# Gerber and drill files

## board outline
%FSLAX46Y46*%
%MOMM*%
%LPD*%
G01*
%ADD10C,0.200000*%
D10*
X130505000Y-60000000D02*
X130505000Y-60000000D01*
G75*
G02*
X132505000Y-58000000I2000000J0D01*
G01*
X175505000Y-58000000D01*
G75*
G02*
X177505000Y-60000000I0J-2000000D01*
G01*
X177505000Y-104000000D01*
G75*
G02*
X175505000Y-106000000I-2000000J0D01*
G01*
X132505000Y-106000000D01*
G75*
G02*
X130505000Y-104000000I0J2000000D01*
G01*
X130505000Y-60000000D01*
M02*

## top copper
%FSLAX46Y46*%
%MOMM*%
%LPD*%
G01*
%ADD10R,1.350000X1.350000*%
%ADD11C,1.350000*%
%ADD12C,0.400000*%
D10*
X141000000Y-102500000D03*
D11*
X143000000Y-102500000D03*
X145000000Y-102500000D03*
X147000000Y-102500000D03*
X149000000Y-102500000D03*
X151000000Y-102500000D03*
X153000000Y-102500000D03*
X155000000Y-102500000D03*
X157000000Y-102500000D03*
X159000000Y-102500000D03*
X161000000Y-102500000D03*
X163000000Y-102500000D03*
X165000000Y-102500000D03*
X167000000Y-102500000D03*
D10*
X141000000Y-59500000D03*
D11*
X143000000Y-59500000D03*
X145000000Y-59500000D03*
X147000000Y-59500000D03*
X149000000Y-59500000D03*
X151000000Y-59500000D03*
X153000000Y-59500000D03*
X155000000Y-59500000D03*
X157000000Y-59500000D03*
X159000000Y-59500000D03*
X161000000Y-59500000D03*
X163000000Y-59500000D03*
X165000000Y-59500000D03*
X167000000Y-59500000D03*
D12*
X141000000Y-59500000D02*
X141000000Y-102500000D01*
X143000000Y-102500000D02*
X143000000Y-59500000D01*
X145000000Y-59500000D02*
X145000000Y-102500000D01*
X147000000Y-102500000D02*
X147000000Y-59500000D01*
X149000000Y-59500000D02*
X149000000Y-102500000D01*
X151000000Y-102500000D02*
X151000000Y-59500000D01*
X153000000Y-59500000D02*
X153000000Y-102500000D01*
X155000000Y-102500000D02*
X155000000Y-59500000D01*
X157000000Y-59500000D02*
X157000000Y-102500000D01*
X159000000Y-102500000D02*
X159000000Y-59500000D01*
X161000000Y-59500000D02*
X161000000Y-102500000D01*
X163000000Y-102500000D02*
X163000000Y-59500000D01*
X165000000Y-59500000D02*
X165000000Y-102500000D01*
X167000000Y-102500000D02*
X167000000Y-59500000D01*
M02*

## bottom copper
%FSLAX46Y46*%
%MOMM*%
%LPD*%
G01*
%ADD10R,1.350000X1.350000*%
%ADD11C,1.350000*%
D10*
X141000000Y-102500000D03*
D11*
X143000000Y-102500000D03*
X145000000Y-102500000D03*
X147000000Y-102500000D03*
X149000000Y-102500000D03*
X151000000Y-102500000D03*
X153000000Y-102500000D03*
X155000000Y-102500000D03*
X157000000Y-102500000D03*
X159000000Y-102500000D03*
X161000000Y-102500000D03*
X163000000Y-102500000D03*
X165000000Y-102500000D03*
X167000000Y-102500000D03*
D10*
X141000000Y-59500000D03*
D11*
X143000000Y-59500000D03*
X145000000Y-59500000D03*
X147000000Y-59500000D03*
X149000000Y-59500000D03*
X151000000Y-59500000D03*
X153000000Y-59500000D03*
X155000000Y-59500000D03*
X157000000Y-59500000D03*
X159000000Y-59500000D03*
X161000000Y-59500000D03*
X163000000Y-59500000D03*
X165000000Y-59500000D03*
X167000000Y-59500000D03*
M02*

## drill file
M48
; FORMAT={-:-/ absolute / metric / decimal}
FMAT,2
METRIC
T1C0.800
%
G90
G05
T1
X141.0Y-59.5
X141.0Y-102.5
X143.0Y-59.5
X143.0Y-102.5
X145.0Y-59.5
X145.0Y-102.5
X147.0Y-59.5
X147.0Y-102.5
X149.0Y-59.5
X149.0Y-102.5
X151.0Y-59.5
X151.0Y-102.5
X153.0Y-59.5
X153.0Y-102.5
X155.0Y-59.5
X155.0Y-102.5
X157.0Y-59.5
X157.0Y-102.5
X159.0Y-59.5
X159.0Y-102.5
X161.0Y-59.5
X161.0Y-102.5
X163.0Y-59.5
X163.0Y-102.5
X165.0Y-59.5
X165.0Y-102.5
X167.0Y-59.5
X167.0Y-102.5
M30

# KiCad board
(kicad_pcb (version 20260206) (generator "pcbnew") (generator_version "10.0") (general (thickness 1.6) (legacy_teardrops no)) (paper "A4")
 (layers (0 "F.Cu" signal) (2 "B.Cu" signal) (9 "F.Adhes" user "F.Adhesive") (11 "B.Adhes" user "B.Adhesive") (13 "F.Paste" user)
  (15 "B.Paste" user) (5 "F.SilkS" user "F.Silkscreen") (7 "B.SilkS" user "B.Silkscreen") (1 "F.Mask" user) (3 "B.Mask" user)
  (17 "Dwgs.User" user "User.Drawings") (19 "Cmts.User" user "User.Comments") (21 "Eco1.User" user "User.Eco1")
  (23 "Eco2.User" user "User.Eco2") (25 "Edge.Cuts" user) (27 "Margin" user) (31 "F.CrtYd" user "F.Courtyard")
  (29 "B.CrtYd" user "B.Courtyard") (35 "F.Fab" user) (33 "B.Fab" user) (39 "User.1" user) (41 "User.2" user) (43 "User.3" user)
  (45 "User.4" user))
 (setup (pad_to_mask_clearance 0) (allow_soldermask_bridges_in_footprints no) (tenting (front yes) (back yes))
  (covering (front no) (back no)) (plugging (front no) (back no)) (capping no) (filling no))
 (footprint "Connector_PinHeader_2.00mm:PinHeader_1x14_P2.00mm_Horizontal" (layer "F.Cu") (at 167 102.5 -90)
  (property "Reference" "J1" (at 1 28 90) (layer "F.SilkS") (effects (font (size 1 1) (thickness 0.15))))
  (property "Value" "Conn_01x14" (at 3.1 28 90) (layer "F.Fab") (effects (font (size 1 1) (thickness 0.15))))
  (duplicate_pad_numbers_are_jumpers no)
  (pad "1" thru_hole rect (at 0 26 270) (size 1.35 1.35) (drill 0.8) (layers "*.Cu" "*.Mask") (remove_unused_layers no)
   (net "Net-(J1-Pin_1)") (thermal_bridge_angle 45))
  (pad "2" thru_hole circle (at 0 24 270) (size 1.35 1.35) (drill 0.8) (layers "*.Cu" "*.Mask") (remove_unused_layers no)
   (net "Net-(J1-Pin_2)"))
  (pad "3" thru_hole circle (at 0 22 270) (size 1.35 1.35) (drill 0.8) (layers "*.Cu" "*.Mask") (remove_unused_layers no)
   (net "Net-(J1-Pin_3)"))
  (pad "4" thru_hole circle (at 0 20 270) (size 1.35 1.35) (drill 0.8) (layers "*.Cu" "*.Mask") (remove_unused_layers no)
   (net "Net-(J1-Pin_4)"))
  (pad "5" thru_hole circle (at 0 18 270) (size 1.35 1.35) (drill 0.8) (layers "*.Cu" "*.Mask") (remove_unused_layers no)
   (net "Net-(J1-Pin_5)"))
  (pad "6" thru_hole circle (at 0 16 270) (size 1.35 1.35) (drill 0.8) (layers "*.Cu" "*.Mask") (remove_unused_layers no)
   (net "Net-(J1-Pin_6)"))
  (pad "7" thru_hole circle (at 0 14 270) (size 1.35 1.35) (drill 0.8) (layers "*.Cu" "*.Mask") (remove_unused_layers no)
   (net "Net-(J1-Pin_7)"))
  (pad "8" thru_hole circle (at 0 12 270) (size 1.35 1.35) (drill 0.8) (layers "*.Cu" "*.Mask") (remove_unused_layers no)
   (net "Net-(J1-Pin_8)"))
  (pad "9" thru_hole circle (at 0 10 270) (size 1.35 1.35) (drill 0.8) (layers "*.Cu" "*.Mask") (remove_unused_layers no)
   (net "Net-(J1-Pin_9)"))
  (pad "10" thru_hole circle (at 0 8 270) (size 1.35 1.35) (drill 0.8) (layers "*.Cu" "*.Mask") (remove_unused_layers no)
   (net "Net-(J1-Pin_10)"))
  (pad "11" thru_hole circle (at 0 6 270) (size 1.35 1.35) (drill 0.8) (layers "*.Cu" "*.Mask") (remove_unused_layers no)
   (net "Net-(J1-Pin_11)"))
  (pad "12" thru_hole circle (at 0 4 270) (size 1.35 1.35) (drill 0.8) (layers "*.Cu" "*.Mask") (remove_unused_layers no)
   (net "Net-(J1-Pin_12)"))
  (pad "13" thru_hole circle (at 0 2 270) (size 1.35 1.35) (drill 0.8) (layers "*.Cu" "*.Mask") (remove_unused_layers no)
   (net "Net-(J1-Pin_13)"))
  (pad "14" thru_hole circle (at 0 0 270) (size 1.35 1.35) (drill 0.8) (layers "*.Cu" "*.Mask") (remove_unused_layers no)
   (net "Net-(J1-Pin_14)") (thermal_bridge_angle 90)))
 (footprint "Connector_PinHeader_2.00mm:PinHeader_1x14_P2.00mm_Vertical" (layer "F.Cu") (at 141 59.5 90)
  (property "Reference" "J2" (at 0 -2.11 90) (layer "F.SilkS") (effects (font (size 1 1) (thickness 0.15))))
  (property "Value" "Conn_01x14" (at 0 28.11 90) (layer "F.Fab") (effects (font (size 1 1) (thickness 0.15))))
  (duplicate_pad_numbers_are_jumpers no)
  (pad "1" thru_hole rect (at 0 0 90) (size 1.35 1.35) (drill 0.8) (layers "*.Cu" "*.Mask") (remove_unused_layers no) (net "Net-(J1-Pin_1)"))
  (pad "2" thru_hole circle (at 0 2 90) (size 1.35 1.35) (drill 0.8) (layers "*.Cu" "*.Mask") (remove_unused_layers no)
   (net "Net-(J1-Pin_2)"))
  (pad "3" thru_hole circle (at 0 4 90) (size 1.35 1.35) (drill 0.8) (layers "*.Cu" "*.Mask") (remove_unused_layers no)
   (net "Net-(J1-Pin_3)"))
  (pad "4" thru_hole circle (at 0 6 90) (size 1.35 1.35) (drill 0.8) (layers "*.Cu" "*.Mask") (remove_unused_layers no)
   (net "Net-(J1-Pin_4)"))
  (pad "5" thru_hole circle (at 0 8 90) (size 1.35 1.35) (drill 0.8) (layers "*.Cu" "*.Mask") (remove_unused_layers no)
   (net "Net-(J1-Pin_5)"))
  (pad "6" thru_hole circle (at 0 10 90) (size 1.35 1.35) (drill 0.8) (layers "*.Cu" "*.Mask") (remove_unused_layers no)
   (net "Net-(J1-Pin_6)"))
  (pad "7" thru_hole circle (at 0 12 90) (size 1.35 1.35) (drill 0.8) (layers "*.Cu" "*.Mask") (remove_unused_layers no)
   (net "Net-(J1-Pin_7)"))
  (pad "8" thru_hole circle (at 0 14 90) (size 1.35 1.35) (drill 0.8) (layers "*.Cu" "*.Mask") (remove_unused_layers no)
   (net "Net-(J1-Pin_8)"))
  (pad "9" thru_hole circle (at 0 16 90) (size 1.35 1.35) (drill 0.8) (layers "*.Cu" "*.Mask") (remove_unused_layers no)
   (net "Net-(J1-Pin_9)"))
  (pad "10" thru_hole circle (at 0 18 90) (size 1.35 1.35) (drill 0.8) (layers "*.Cu" "*.Mask") (remove_unused_layers no)
   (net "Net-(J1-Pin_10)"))
  (pad "11" thru_hole circle (at 0 20 90) (size 1.35 1.35) (drill 0.8) (layers "*.Cu" "*.Mask") (remove_unused_layers no)
   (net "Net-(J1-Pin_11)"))
  (pad "12" thru_hole circle (at 0 22 90) (size 1.35 1.35) (drill 0.8) (layers "*.Cu" "*.Mask") (remove_unused_layers no)
   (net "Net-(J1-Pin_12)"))
  (pad "13" thru_hole circle (at 0 24 90) (size 1.35 1.35) (drill 0.8) (layers "*.Cu" "*.Mask") (remove_unused_layers no)
   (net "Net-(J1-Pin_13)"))
  (pad "14" thru_hole circle (at 0 26 90) (size 1.35 1.35) (drill 0.8) (layers "*.Cu" "*.Mask") (remove_unused_layers no)
   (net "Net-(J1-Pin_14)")))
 (gr_rect (start 130.505 58) (end 177.505 106) (radius 2) (stroke (width 0.2) (type solid)) (fill no) (layer "Edge.Cuts"))
 (segment (start 141 59.5) (end 141 102.5) (width 0.4) (layer "F.Cu") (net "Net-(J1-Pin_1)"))
 (segment (start 143 102.5) (end 143 59.5) (width 0.4) (layer "F.Cu") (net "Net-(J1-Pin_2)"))
 (segment (start 145 59.5) (end 145 102.5) (width 0.4) (layer "F.Cu") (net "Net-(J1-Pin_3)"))
 (segment (start 147 102.5) (end 147 59.5) (width 0.4) (layer "F.Cu") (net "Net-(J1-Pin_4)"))
 (segment (start 149 59.5) (end 149 102.5) (width 0.4) (layer "F.Cu") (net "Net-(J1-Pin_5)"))
 (segment (start 151 102.5) (end 151 59.5) (width 0.4) (layer "F.Cu") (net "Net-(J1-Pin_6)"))
 (segment (start 153 59.5) (end 153 102.5) (width 0.4) (layer "F.Cu") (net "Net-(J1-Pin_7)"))
 (segment (start 155 102.5) (end 155 59.5) (width 0.4) (layer "F.Cu") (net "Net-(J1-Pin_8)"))
 (segment (start 157 59.5) (end 157 102.5) (width 0.4) (layer "F.Cu") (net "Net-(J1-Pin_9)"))
 (segment (start 159 102.5) (end 159 59.5) (width 0.4) (layer "F.Cu") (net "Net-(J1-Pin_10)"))
 (segment (start 161 59.5) (end 161 102.5) (width 0.4) (layer "F.Cu") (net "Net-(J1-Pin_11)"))
 (segment (start 163 102.5) (end 163 59.5) (width 0.4) (layer "F.Cu") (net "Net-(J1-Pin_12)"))
 (segment (start 165 59.5) (end 165 102.5) (width 0.4) (layer "F.Cu") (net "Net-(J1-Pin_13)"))
 (segment (start 167 102.5) (end 167 59.5) (width 0.4) (layer "F.Cu") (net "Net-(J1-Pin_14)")))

